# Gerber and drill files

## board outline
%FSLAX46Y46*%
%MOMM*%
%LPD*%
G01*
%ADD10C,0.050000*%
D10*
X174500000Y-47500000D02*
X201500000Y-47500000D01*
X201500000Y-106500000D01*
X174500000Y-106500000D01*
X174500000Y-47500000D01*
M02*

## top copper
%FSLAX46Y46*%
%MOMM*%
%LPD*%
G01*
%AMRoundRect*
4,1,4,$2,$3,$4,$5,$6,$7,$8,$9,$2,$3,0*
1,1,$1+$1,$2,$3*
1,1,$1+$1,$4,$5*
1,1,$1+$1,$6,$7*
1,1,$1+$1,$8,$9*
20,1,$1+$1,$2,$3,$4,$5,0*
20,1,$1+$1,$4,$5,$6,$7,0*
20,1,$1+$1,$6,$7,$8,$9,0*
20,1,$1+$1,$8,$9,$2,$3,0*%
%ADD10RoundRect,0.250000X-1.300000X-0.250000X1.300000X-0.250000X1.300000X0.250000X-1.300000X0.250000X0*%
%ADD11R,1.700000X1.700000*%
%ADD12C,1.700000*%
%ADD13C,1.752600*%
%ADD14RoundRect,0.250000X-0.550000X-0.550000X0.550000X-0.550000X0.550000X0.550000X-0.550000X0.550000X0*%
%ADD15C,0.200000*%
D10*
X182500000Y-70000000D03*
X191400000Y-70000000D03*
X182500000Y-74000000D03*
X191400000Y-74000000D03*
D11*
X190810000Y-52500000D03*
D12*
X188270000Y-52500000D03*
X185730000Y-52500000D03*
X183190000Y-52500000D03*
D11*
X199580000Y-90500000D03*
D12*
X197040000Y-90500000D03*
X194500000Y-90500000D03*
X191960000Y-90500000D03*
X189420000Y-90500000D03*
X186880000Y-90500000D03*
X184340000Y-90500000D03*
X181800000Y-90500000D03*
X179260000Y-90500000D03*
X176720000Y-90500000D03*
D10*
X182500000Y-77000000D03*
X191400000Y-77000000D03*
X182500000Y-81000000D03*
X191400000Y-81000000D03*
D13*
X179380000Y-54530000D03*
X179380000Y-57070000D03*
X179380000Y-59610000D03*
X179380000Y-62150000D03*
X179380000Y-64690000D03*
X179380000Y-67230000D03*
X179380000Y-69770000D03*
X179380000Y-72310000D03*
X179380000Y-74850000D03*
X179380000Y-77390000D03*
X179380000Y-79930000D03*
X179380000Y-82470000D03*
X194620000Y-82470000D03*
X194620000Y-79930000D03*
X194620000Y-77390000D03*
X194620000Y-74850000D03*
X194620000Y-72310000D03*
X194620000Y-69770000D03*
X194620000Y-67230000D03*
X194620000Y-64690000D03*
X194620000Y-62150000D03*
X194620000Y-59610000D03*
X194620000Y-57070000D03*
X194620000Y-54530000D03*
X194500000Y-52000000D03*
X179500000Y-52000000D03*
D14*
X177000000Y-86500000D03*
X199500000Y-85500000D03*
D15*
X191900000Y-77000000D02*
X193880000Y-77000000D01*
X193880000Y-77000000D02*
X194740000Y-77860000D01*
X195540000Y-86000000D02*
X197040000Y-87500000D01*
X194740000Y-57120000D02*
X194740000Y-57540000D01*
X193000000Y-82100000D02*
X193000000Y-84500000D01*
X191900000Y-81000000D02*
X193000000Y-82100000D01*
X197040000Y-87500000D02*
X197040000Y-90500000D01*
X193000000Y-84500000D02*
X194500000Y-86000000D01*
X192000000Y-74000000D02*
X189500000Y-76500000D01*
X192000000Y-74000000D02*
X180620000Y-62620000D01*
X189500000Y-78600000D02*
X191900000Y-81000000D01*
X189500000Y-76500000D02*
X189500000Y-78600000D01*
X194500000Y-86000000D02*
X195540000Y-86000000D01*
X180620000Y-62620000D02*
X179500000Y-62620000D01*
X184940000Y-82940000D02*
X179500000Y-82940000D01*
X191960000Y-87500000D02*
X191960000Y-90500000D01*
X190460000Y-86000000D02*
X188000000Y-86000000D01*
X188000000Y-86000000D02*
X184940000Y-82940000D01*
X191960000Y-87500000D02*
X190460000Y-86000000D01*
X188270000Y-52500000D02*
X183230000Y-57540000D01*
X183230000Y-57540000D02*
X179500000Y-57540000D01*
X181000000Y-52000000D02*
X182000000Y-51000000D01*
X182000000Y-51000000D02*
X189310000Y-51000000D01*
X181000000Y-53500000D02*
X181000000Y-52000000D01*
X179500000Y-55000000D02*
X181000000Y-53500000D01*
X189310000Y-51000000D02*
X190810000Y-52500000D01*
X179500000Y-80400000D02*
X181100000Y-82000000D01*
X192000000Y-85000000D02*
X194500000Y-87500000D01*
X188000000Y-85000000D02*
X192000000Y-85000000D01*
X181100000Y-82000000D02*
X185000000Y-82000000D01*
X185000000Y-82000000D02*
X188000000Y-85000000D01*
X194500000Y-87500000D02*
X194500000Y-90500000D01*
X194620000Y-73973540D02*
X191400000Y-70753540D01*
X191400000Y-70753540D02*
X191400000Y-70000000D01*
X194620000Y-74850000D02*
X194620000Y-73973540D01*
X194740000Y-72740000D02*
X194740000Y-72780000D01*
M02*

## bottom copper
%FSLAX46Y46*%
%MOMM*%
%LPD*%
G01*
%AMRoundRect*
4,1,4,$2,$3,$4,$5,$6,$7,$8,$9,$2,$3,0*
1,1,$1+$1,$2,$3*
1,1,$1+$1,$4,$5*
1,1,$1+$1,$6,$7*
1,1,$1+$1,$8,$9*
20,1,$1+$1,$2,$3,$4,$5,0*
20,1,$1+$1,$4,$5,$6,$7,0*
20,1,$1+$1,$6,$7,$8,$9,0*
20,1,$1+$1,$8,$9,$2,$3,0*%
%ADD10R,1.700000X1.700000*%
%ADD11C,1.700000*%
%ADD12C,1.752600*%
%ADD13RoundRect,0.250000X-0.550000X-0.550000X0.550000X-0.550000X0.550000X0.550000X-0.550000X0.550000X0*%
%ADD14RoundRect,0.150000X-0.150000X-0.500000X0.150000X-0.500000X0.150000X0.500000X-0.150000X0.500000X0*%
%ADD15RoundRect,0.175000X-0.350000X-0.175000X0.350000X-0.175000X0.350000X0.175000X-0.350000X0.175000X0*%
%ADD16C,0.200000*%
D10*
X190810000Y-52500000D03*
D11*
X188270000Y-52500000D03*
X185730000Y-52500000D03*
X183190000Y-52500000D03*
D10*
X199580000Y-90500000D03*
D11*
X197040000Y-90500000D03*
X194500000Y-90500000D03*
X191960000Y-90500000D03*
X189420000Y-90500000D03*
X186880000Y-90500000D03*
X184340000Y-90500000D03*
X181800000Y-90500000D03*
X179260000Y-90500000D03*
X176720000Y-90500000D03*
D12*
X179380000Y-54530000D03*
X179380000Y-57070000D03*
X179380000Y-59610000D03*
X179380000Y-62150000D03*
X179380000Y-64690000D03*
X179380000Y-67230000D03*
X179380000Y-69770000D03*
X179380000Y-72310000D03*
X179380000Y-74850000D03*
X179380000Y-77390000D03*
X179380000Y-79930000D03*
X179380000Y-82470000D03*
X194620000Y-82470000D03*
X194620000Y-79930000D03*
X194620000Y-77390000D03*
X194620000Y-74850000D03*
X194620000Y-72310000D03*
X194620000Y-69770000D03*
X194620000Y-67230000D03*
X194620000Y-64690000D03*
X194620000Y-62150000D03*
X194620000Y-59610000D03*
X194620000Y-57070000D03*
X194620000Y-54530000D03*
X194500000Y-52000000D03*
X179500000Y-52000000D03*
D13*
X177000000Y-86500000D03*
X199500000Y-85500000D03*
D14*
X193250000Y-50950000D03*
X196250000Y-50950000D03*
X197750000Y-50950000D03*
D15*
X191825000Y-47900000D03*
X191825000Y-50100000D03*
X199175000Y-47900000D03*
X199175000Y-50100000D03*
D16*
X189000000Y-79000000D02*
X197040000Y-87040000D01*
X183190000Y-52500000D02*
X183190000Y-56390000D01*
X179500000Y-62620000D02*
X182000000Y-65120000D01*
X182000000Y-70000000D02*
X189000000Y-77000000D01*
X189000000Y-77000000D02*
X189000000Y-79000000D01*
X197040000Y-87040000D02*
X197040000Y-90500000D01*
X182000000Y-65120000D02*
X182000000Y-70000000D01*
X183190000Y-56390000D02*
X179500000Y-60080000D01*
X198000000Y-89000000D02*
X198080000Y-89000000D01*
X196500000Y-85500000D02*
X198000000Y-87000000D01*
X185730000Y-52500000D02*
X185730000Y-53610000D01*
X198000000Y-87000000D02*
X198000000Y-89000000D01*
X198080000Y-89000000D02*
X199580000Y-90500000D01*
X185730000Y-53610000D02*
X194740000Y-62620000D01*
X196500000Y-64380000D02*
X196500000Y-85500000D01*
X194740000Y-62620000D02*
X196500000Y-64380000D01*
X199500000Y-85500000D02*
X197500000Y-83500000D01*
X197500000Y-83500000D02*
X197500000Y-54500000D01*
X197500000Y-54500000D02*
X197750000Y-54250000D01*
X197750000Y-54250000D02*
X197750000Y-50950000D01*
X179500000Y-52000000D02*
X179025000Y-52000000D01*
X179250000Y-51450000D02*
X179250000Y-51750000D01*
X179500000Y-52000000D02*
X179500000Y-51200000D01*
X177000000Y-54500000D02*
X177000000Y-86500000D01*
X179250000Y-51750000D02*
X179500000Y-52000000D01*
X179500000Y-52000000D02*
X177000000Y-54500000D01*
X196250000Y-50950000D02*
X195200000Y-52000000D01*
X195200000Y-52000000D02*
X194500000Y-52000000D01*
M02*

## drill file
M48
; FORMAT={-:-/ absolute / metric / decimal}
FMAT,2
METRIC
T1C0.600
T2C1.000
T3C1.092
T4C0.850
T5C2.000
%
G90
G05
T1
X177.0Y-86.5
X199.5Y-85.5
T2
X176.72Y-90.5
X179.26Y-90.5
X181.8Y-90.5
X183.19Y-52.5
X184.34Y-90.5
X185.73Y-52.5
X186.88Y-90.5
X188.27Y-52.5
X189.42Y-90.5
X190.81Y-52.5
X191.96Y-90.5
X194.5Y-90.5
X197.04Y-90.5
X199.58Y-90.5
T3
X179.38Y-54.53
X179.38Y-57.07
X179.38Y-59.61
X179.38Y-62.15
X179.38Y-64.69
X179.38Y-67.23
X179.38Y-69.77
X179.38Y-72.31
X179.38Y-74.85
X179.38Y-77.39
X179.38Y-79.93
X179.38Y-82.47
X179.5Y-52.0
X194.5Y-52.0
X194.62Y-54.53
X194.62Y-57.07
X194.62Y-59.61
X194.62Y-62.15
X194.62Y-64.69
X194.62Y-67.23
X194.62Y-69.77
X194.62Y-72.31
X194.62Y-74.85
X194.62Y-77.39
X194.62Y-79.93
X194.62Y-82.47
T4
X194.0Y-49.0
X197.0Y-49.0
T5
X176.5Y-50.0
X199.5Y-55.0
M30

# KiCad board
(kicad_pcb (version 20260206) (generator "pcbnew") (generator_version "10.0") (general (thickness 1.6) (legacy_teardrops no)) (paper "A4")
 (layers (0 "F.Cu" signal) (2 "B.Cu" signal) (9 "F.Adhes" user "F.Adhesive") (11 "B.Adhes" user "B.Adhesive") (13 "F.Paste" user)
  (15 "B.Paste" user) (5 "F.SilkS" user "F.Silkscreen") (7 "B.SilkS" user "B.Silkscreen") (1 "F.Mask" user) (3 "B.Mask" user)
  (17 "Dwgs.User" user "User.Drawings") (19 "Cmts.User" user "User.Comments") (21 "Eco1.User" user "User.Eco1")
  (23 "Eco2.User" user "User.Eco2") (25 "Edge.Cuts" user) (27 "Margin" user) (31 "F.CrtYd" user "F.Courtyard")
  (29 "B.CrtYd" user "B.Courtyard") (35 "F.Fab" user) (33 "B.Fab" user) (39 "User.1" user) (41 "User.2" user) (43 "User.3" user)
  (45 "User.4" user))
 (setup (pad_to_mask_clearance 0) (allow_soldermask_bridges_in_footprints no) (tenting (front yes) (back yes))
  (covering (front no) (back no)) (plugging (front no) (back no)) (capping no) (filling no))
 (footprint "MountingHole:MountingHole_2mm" (layer "F.Cu") (at 176.5 50)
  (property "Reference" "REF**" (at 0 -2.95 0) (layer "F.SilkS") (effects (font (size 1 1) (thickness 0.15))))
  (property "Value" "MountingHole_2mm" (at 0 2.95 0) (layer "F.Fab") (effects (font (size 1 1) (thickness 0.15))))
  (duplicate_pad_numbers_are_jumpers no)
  (pad "" np_thru_hole circle (at 0 0) (size 2 2) (drill 2) (layers "*.Cu" "*.Mask")))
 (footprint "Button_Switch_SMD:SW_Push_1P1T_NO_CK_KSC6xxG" (layer "F.Cu") (at 186.95 72)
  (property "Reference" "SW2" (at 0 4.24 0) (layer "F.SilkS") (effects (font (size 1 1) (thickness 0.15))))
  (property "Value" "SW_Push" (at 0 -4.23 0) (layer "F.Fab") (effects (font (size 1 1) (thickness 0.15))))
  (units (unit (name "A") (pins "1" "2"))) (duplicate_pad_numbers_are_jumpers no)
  (pad "1" smd roundrect (at -4.45 -2) (size 3.1 1) (layers "F.Cu" "F.Mask" "F.Paste") (roundrect_rratio 0.25) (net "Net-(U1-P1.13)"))
  (pad "1" smd roundrect (at 4.45 -2) (size 3.1 1) (layers "F.Cu" "F.Mask" "F.Paste") (roundrect_rratio 0.25) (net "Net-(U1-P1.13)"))
  (pad "2" smd roundrect (at -4.45 2) (size 3.1 1) (layers "F.Cu" "F.Mask" "F.Paste") (roundrect_rratio 0.25) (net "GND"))
  (pad "2" smd roundrect (at 4.45 2) (size 3.1 1) (layers "F.Cu" "F.Mask" "F.Paste") (roundrect_rratio 0.25) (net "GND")))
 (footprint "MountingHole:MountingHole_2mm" (layer "F.Cu") (at 199.5 55)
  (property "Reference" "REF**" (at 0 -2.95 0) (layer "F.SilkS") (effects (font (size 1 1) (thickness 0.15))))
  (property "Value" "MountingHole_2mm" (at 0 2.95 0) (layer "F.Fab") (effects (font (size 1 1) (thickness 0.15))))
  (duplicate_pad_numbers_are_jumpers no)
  (pad "" np_thru_hole circle (at 0 0) (size 2 2) (drill 2) (layers "*.Cu" "*.Mask")))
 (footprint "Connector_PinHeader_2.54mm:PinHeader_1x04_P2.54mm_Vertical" (layer "F.Cu") (at 190.81 52.5 -90)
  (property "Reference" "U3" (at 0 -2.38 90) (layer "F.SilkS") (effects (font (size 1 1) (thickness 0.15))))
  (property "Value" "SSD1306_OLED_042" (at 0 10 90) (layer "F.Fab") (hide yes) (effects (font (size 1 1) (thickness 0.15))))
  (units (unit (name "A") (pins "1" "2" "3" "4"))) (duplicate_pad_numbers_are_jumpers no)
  (pad "1" thru_hole rect (at 0 0 270) (size 1.7 1.7) (drill 1) (layers "*.Cu" "*.Mask") (remove_unused_layers no)
   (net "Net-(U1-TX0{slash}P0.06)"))
  (pad "2" thru_hole circle (at 0 2.54 270) (size 1.7 1.7) (drill 1) (layers "*.Cu" "*.Mask") (remove_unused_layers no)
   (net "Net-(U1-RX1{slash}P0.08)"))
  (pad "3" thru_hole circle (at 0 5.08 270) (size 1.7 1.7) (drill 1) (layers "*.Cu" "*.Mask") (remove_unused_layers no) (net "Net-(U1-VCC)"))
  (pad "4" thru_hole circle (at 0 7.62 270) (size 1.7 1.7) (drill 1) (layers "*.Cu" "*.Mask") (remove_unused_layers no) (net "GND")))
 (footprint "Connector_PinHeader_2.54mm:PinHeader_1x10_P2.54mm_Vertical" (layer "F.Cu") (at 199.58 90.5 -90)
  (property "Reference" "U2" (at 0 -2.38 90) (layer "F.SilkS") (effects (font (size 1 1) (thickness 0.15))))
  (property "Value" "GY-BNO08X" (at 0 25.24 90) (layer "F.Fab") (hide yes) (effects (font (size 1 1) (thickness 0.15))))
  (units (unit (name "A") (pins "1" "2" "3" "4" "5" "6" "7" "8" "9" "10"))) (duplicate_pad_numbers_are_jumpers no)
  (pad "1" thru_hole rect (at 0 0 270) (size 1.7 1.7) (drill 1) (layers "*.Cu" "*.Mask") (remove_unused_layers no) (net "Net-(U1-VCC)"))
  (pad "2" thru_hole circle (at 0 2.54 270) (size 1.7 1.7) (drill 1) (layers "*.Cu" "*.Mask") (remove_unused_layers no) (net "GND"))
  (pad "3" thru_hole circle (at 0 5.08 270) (size 1.7 1.7) (drill 1) (layers "*.Cu" "*.Mask") (remove_unused_layers no)
   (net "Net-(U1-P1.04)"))
  (pad "4" thru_hole circle (at 0 7.62 270) (size 1.7 1.7) (drill 1) (layers "*.Cu" "*.Mask") (remove_unused_layers no)
   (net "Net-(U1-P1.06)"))
  (pad "5" thru_hole circle (at 0 10.16 270) (size 1.7 1.7) (drill 1) (layers "*.Cu" "*.Mask") (remove_unused_layers no)
   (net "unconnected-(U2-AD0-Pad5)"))
  (pad "6" thru_hole circle (at 0 12.7 270) (size 1.7 1.7) (drill 1) (layers "*.Cu" "*.Mask") (remove_unused_layers no)
   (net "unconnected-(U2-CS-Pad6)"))
  (pad "7" thru_hole circle (at 0 15.24 270) (size 1.7 1.7) (drill 1) (layers "*.Cu" "*.Mask") (remove_unused_layers no)
   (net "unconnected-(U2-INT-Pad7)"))
  (pad "8" thru_hole circle (at 0 17.78 270) (size 1.7 1.7) (drill 1) (layers "*.Cu" "*.Mask") (remove_unused_layers no)
   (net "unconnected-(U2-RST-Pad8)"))
  (pad "9" thru_hole circle (at 0 20.32 270) (size 1.7 1.7) (drill 1) (layers "*.Cu" "*.Mask") (remove_unused_layers no)
   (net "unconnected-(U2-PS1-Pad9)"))
  (pad "10" thru_hole circle (at 0 22.86 270) (size 1.7 1.7) (drill 1) (layers "*.Cu" "*.Mask") (remove_unused_layers no)
   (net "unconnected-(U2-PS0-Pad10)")))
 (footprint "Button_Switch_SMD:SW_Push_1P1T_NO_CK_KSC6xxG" (layer "F.Cu") (at 186.95 79)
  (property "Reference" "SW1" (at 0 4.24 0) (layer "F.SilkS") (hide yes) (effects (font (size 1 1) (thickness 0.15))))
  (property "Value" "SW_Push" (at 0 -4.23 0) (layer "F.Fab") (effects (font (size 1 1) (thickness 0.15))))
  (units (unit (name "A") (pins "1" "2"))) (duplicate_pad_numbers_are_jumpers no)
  (pad "1" smd roundrect (at -4.45 -2) (size 3.1 1) (layers "F.Cu" "F.Mask" "F.Paste") (roundrect_rratio 0.25) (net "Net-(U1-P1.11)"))
  (pad "1" smd roundrect (at 4.45 -2) (size 3.1 1) (layers "F.Cu" "F.Mask" "F.Paste") (roundrect_rratio 0.25) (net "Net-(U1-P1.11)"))
  (pad "2" smd roundrect (at -4.45 2) (size 3.1 1) (layers "F.Cu" "F.Mask" "F.Paste") (roundrect_rratio 0.25) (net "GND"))
  (pad "2" smd roundrect (at 4.45 2) (size 3.1 1) (layers "F.Cu" "F.Mask" "F.Paste") (roundrect_rratio 0.25) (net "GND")))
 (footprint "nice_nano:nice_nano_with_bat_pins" (layer "F.Cu") (at 187 68.5 -90)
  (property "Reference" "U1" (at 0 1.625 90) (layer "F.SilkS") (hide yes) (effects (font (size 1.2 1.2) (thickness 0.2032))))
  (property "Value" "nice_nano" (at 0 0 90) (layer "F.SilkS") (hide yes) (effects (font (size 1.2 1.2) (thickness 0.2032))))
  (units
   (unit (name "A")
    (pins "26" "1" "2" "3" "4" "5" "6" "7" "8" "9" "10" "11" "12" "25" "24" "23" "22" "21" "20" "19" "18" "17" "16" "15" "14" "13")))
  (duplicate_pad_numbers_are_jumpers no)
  (pad "1" thru_hole circle (at -13.97 7.62 270) (size 1.7526 1.7526) (drill 1.0922) (layers "*.Cu" "*.SilkS" "*.Mask")
   (remove_unused_layers no) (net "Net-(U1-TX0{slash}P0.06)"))
  (pad "2" thru_hole circle (at -11.43 7.62 270) (size 1.7526 1.7526) (drill 1.0922) (layers "*.Cu" "*.SilkS" "*.Mask")
   (remove_unused_layers no) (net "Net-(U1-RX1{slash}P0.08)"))
  (pad "3" thru_hole circle (at -8.89 7.62 270) (size 1.7526 1.7526) (drill 1.0922) (layers "*.Cu" "*.SilkS" "*.Mask")
   (remove_unused_layers no) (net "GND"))
  (pad "4" thru_hole circle (at -6.35 7.62 270) (size 1.7526 1.7526) (drill 1.0922) (layers "*.Cu" "*.SilkS" "*.Mask")
   (remove_unused_layers no) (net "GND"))
  (pad "5" thru_hole circle (at -3.81 7.62 270) (size 1.7526 1.7526) (drill 1.0922) (layers "*.Cu" "*.SilkS" "*.Mask")
   (remove_unused_layers no) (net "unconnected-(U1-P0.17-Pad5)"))
  (pad "6" thru_hole circle (at -1.27 7.62 270) (size 1.7526 1.7526) (drill 1.0922) (layers "*.Cu" "*.SilkS" "*.Mask")
   (remove_unused_layers no) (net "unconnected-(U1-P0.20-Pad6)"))
  (pad "7" thru_hole circle (at 1.27 7.62 270) (size 1.7526 1.7526) (drill 1.0922) (layers "*.Cu" "*.SilkS" "*.Mask")
   (remove_unused_layers no) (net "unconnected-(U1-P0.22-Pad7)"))
  (pad "8" thru_hole circle (at 3.81 7.62 270) (size 1.7526 1.7526) (drill 1.0922) (layers "*.Cu" "*.SilkS" "*.Mask")
   (remove_unused_layers no) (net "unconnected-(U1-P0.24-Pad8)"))
  (pad "9" thru_hole circle (at 6.35 7.62 270) (size 1.7526 1.7526) (drill 1.0922) (layers "*.Cu" "*.SilkS" "*.Mask")
   (remove_unused_layers no) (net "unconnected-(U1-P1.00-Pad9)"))
  (pad "10" thru_hole circle (at 8.89 7.62 270) (size 1.7526 1.7526) (drill 1.0922) (layers "*.Cu" "*.SilkS" "*.Mask")
   (remove_unused_layers no) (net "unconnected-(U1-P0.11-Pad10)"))
  (pad "11" thru_hole circle (at 11.43 7.62 270) (size 1.7526 1.7526) (drill 1.0922) (layers "*.Cu" "*.SilkS" "*.Mask")
   (remove_unused_layers no) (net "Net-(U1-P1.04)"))
  (pad "12" thru_hole circle (at 13.97 7.62 270) (size 1.7526 1.7526) (drill 1.0922) (layers "*.Cu" "*.SilkS" "*.Mask")
   (remove_unused_layers no) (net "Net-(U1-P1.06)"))
  (pad "13" thru_hole circle (at 13.97 -7.62 270) (size 1.7526 1.7526) (drill 1.0922) (layers "*.Cu" "*.SilkS" "*.Mask")
   (remove_unused_layers no) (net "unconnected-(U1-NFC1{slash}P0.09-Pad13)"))
  (pad "14" thru_hole circle (at 11.43 -7.62 270) (size 1.7526 1.7526) (drill 1.0922) (layers "*.Cu" "*.SilkS" "*.Mask")
   (remove_unused_layers no) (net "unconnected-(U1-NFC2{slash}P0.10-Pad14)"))
  (pad "15" thru_hole circle (at 8.89 -7.62 270) (size 1.7526 1.7526) (drill 1.0922) (layers "*.Cu" "*.SilkS" "*.Mask")
   (remove_unused_layers no) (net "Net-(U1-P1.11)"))
  (pad "16" thru_hole circle (at 6.35 -7.62 270) (size 1.7526 1.7526) (drill 1.0922) (layers "*.Cu" "*.SilkS" "*.Mask")
   (remove_unused_layers no) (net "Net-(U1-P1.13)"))
  (pad "17" thru_hole circle (at 3.81 -7.62 270) (size 1.7526 1.7526) (drill 1.0922) (layers "*.Cu" "*.SilkS" "*.Mask")
   (remove_unused_layers no) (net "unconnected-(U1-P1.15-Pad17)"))
  (pad "18" thru_hole circle (at 1.27 -7.62 270) (size 1.7526 1.7526) (drill 1.0922) (layers "*.Cu" "*.SilkS" "*.Mask")
   (remove_unused_layers no) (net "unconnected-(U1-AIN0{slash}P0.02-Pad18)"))
  (pad "19" thru_hole circle (at -1.27 -7.62 270) (size 1.7526 1.7526) (drill 1.0922) (layers "*.Cu" "*.SilkS" "*.Mask")
   (remove_unused_layers no) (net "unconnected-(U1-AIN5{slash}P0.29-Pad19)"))
  (pad "20" thru_hole circle (at -3.81 -7.62 270) (size 1.7526 1.7526) (drill 1.0922) (layers "*.Cu" "*.SilkS" "*.Mask")
   (remove_unused_layers no) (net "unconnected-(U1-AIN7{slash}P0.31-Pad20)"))
  (pad "21" thru_hole circle (at -6.35 -7.62 270) (size 1.7526 1.7526) (drill 1.0922) (layers "*.Cu" "*.SilkS" "*.Mask")
   (remove_unused_layers no) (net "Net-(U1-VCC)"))
  (pad "22" thru_hole circle (at -8.89 -7.62 270) (size 1.7526 1.7526) (drill 1.0922) (layers "*.Cu" "*.SilkS" "*.Mask")
   (remove_unused_layers no) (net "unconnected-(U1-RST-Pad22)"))
  (pad "23" thru_hole circle (at -11.43 -7.62 270) (size 1.7526 1.7526) (drill 1.0922) (layers "*.Cu" "*.SilkS" "*.Mask")
   (remove_unused_layers no) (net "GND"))
  (pad "24" thru_hole circle (at -13.97 -7.62 270) (size 1.7526 1.7526) (drill 1.0922) (layers "*.Cu" "*.SilkS" "*.Mask")
   (remove_unused_layers no) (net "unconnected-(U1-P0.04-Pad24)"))
  (pad "25" thru_hole circle (at -16.5 -7.5 270) (size 1.7526 1.7526) (drill 1.0922) (layers "*.Cu" "*.SilkS" "*.Mask")
   (remove_unused_layers no) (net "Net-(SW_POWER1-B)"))
  (pad "26" thru_hole circle (at -16.5 7.5 270) (size 1.7526 1.7526) (drill 1.0922) (layers "*.Cu" "*.SilkS" "*.Mask")
   (remove_unused_layers no) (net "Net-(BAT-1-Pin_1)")))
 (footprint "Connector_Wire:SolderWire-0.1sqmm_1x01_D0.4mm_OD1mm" (layer "B.Cu") (at 177 86.5)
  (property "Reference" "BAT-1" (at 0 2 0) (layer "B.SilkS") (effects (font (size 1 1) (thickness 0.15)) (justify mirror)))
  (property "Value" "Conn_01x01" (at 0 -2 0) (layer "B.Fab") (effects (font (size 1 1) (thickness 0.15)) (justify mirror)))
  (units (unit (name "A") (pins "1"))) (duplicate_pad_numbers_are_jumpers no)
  (pad "1" thru_hole roundrect (at 0 0) (size 1.6 1.6) (drill 0.6) (layers "*.Cu" "*.Mask") (remove_unused_layers no)
   (roundrect_rratio 0.15625) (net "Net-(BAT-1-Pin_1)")))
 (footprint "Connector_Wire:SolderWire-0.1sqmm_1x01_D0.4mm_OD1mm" (layer "B.Cu") (at 199.5 85.5)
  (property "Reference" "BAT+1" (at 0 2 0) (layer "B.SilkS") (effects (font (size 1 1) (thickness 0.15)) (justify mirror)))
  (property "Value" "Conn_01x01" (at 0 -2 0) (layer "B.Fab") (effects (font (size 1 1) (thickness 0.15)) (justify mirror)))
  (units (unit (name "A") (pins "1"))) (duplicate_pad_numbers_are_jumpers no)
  (pad "1" thru_hole roundrect (at 0 0) (size 1.6 1.6) (drill 0.6) (layers "*.Cu" "*.Mask") (remove_unused_layers no)
   (roundrect_rratio 0.15625) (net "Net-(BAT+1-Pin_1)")))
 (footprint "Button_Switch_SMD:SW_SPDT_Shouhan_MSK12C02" (layer "B.Cu") (at 195.5 49)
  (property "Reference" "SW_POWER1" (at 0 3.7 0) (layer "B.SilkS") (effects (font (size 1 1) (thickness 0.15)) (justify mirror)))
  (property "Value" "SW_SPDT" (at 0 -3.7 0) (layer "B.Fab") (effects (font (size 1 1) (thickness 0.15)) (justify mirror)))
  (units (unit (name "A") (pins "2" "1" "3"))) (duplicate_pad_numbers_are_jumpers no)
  (pad "" np_thru_hole circle (at -1.5 0) (size 0.85 0.85) (drill 0.85) (layers "*.Mask"))
  (pad "" np_thru_hole circle (at 1.5 0) (size 0.85 0.85) (drill 0.85) (layers "*.Mask"))
  (pad "1" smd roundrect (at -2.25 1.95) (size 0.6 1.3) (layers "B.Cu" "B.Mask" "B.Paste") (roundrect_rratio 0.25)
   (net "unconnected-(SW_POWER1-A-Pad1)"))
  (pad "2" smd roundrect (at 0.75 1.95) (size 0.6 1.3) (layers "B.Cu" "B.Mask" "B.Paste") (roundrect_rratio 0.25) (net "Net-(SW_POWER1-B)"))
  (pad "3" smd roundrect (at 2.25 1.95) (size 0.6 1.3) (layers "B.Cu" "B.Mask" "B.Paste") (roundrect_rratio 0.25) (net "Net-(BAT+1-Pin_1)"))
  (pad "SH" smd roundrect (at -3.675 -1.1) (size 1.05 0.7) (layers "B.Cu" "B.Mask" "B.Paste") (roundrect_rratio 0.25))
  (pad "SH" smd roundrect (at -3.675 1.1) (size 1.05 0.7) (layers "B.Cu" "B.Mask" "B.Paste") (roundrect_rratio 0.25))
  (pad "SH" smd roundrect (at 3.675 -1.1) (size 1.05 0.7) (layers "B.Cu" "B.Mask" "B.Paste") (roundrect_rratio 0.25))
  (pad "SH" smd roundrect (at 3.675 1.1) (size 1.05 0.7) (layers "B.Cu" "B.Mask" "B.Paste") (roundrect_rratio 0.25)))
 (gr_rect (start 174.5 47.5) (end 201.5 106.5) (stroke (width 0.05) (type default)) (fill no) (layer "Edge.Cuts"))
 (segment (start 191.9 77) (end 193.88 77) (width 0.2) (layer "F.Cu") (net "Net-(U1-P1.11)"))
 (segment (start 193.88 77) (end 194.74 77.86) (width 0.2) (layer "F.Cu") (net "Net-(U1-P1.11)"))
 (segment (start 195.54 86) (end 197.04 87.5) (width 0.2) (layer "F.Cu") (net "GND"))
 (segment (start 194.74 57.12) (end 194.74 57.54) (width 0.2) (layer "F.Cu") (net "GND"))
 (segment (start 193 82.1) (end 193 84.5) (width 0.2) (layer "F.Cu") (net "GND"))
 (segment (start 191.9 81) (end 193 82.1) (width 0.2) (layer "F.Cu") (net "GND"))
 (segment (start 197.04 87.5) (end 197.04 90.5) (width 0.2) (layer "F.Cu") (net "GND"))
 (segment (start 193 84.5) (end 194.5 86) (width 0.2) (layer "F.Cu") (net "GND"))
 (segment (start 192 74) (end 189.5 76.5) (width 0.2) (layer "F.Cu") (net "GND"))
 (segment (start 192 74) (end 180.62 62.62) (width 0.2) (layer "F.Cu") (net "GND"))
 (segment (start 189.5 78.6) (end 191.9 81) (width 0.2) (layer "F.Cu") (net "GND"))
 (segment (start 189.5 76.5) (end 189.5 78.6) (width 0.2) (layer "F.Cu") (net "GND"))
 (segment (start 194.5 86) (end 195.54 86) (width 0.2) (layer "F.Cu") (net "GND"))
 (segment (start 180.62 62.62) (end 179.5 62.62) (width 0.2) (layer "F.Cu") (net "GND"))
 (segment (start 189 79) (end 197.04 87.04) (width 0.2) (layer "B.Cu") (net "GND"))
 (segment (start 183.19 52.5) (end 183.19 56.39) (width 0.2) (layer "B.Cu") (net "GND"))
 (segment (start 179.5 62.62) (end 182 65.12) (width 0.2) (layer "B.Cu") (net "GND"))
 (segment (start 182 70) (end 189 77) (width 0.2) (layer "B.Cu") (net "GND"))
 (segment (start 189 77) (end 189 79) (width 0.2) (layer "B.Cu") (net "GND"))
 (segment (start 197.04 87.04) (end 197.04 90.5) (width 0.2) (layer "B.Cu") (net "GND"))
 (segment (start 182 65.12) (end 182 70) (width 0.2) (layer "B.Cu") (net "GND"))
 (segment (start 183.19 56.39) (end 179.5 60.08) (width 0.2) (layer "B.Cu") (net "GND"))
 (segment (start 184.94 82.94) (end 179.5 82.94) (width 0.2) (layer "F.Cu") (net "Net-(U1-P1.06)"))
 (segment (start 191.96 87.5) (end 191.96 90.5) (width 0.2) (layer "F.Cu") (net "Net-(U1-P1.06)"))
 (segment (start 190.46 86) (end 188 86) (width 0.2) (layer "F.Cu") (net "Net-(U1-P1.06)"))
 (segment (start 188 86) (end 184.94 82.94) (width 0.2) (layer "F.Cu") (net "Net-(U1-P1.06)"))
 (segment (start 191.96 87.5) (end 190.46 86) (width 0.2) (layer "F.Cu") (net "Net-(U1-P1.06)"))
 (segment (start 188.27 52.5) (end 183.23 57.54) (width 0.2) (layer "F.Cu") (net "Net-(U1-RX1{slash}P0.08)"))
 (segment (start 183.23 57.54) (end 179.5 57.54) (width 0.2) (layer "F.Cu") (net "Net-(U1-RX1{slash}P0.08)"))
 (segment (start 198 89) (end 198.08 89) (width 0.2) (layer "B.Cu") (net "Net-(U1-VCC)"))
 (segment (start 196.5 85.5) (end 198 87) (width 0.2) (layer "B.Cu") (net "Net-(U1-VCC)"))
 (segment (start 185.73 52.5) (end 185.73 53.61) (width 0.2) (layer "B.Cu") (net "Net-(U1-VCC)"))
 (segment (start 198 87) (end 198 89) (width 0.2) (layer "B.Cu") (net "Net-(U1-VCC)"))
 (segment (start 198.08 89) (end 199.58 90.5) (width 0.2) (layer "B.Cu") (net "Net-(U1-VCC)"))
 (segment (start 185.73 53.61) (end 194.74 62.62) (width 0.2) (layer "B.Cu") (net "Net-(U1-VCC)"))
 (segment (start 196.5 64.38) (end 196.5 85.5) (width 0.2) (layer "B.Cu") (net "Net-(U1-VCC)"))
 (segment (start 194.74 62.62) (end 196.5 64.38) (width 0.2) (layer "B.Cu") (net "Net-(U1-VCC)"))
 (segment (start 181 52) (end 182 51) (width 0.2) (layer "F.Cu") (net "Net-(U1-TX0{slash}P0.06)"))
 (segment (start 182 51) (end 189.31 51) (width 0.2) (layer "F.Cu") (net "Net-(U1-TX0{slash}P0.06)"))
 (segment (start 181 53.5) (end 181 52) (width 0.2) (layer "F.Cu") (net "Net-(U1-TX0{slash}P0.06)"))
 (segment (start 179.5 55) (end 181 53.5) (width 0.2) (layer "F.Cu") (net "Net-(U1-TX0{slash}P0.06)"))
 (segment (start 189.31 51) (end 190.81 52.5) (width 0.2) (layer "F.Cu") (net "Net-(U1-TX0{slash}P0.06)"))
 (segment (start 179.5 80.4) (end 181.1 82) (width 0.2) (layer "F.Cu") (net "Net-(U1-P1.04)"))
 (segment (start 192 85) (end 194.5 87.5) (width 0.2) (layer "F.Cu") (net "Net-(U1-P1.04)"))
 (segment (start 188 85) (end 192 85) (width 0.2) (layer "F.Cu") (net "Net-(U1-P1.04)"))
 (segment (start 181.1 82) (end 185 82) (width 0.2) (layer "F.Cu") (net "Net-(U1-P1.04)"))
 (segment (start 185 82) (end 188 85) (width 0.2) (layer "F.Cu") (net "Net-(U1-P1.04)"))
 (segment (start 194.5 87.5) (end 194.5 90.5) (width 0.2) (layer "F.Cu") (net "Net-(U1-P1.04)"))
 (segment (start 194.62 73.97354) (end 191.4 70.75354) (width 0.2) (layer "F.Cu") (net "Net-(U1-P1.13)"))
 (segment (start 191.4 70.75354) (end 191.4 70) (width 0.2) (layer "F.Cu") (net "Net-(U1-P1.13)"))
 (segment (start 194.62 74.85) (end 194.62 73.97354) (width 0.2) (layer "F.Cu") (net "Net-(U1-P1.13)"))
 (segment (start 194.74 72.74) (end 194.74 72.78) (width 0.2) (layer "F.Cu") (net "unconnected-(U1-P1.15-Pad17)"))
 (segment (start 199.5 85.5) (end 197.5 83.5) (width 0.2) (layer "B.Cu") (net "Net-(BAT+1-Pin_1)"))
 (segment (start 197.5 83.5) (end 197.5 54.5) (width 0.2) (layer "B.Cu") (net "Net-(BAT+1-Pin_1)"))
 (segment (start 197.5 54.5) (end 197.75 54.25) (width 0.2) (layer "B.Cu") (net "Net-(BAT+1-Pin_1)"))
 (segment (start 197.75 54.25) (end 197.75 50.95) (width 0.2) (layer "B.Cu") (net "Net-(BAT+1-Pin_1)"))
 (segment (start 179.5 52) (end 179.025 52) (width 0.2) (layer "B.Cu") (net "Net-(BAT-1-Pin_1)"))
 (segment (start 179.25 51.45) (end 179.25 51.75) (width 0.2) (layer "B.Cu") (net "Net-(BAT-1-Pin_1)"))
 (segment (start 179.5 52) (end 179.5 51.2) (width 0.2) (layer "B.Cu") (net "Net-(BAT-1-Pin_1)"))
 (segment (start 177 54.5) (end 177 86.5) (width 0.2) (layer "B.Cu") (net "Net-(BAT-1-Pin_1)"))
 (segment (start 179.25 51.75) (end 179.5 52) (width 0.2) (layer "B.Cu") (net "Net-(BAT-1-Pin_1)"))
 (segment (start 179.5 52) (end 177 54.5) (width 0.2) (layer "B.Cu") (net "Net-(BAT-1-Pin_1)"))
 (segment (start 196.25 50.95) (end 195.2 52) (width 0.2) (layer "B.Cu") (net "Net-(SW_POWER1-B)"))
 (segment (start 195.2 52) (end 194.5 52) (width 0.2) (layer "B.Cu") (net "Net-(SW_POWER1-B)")))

